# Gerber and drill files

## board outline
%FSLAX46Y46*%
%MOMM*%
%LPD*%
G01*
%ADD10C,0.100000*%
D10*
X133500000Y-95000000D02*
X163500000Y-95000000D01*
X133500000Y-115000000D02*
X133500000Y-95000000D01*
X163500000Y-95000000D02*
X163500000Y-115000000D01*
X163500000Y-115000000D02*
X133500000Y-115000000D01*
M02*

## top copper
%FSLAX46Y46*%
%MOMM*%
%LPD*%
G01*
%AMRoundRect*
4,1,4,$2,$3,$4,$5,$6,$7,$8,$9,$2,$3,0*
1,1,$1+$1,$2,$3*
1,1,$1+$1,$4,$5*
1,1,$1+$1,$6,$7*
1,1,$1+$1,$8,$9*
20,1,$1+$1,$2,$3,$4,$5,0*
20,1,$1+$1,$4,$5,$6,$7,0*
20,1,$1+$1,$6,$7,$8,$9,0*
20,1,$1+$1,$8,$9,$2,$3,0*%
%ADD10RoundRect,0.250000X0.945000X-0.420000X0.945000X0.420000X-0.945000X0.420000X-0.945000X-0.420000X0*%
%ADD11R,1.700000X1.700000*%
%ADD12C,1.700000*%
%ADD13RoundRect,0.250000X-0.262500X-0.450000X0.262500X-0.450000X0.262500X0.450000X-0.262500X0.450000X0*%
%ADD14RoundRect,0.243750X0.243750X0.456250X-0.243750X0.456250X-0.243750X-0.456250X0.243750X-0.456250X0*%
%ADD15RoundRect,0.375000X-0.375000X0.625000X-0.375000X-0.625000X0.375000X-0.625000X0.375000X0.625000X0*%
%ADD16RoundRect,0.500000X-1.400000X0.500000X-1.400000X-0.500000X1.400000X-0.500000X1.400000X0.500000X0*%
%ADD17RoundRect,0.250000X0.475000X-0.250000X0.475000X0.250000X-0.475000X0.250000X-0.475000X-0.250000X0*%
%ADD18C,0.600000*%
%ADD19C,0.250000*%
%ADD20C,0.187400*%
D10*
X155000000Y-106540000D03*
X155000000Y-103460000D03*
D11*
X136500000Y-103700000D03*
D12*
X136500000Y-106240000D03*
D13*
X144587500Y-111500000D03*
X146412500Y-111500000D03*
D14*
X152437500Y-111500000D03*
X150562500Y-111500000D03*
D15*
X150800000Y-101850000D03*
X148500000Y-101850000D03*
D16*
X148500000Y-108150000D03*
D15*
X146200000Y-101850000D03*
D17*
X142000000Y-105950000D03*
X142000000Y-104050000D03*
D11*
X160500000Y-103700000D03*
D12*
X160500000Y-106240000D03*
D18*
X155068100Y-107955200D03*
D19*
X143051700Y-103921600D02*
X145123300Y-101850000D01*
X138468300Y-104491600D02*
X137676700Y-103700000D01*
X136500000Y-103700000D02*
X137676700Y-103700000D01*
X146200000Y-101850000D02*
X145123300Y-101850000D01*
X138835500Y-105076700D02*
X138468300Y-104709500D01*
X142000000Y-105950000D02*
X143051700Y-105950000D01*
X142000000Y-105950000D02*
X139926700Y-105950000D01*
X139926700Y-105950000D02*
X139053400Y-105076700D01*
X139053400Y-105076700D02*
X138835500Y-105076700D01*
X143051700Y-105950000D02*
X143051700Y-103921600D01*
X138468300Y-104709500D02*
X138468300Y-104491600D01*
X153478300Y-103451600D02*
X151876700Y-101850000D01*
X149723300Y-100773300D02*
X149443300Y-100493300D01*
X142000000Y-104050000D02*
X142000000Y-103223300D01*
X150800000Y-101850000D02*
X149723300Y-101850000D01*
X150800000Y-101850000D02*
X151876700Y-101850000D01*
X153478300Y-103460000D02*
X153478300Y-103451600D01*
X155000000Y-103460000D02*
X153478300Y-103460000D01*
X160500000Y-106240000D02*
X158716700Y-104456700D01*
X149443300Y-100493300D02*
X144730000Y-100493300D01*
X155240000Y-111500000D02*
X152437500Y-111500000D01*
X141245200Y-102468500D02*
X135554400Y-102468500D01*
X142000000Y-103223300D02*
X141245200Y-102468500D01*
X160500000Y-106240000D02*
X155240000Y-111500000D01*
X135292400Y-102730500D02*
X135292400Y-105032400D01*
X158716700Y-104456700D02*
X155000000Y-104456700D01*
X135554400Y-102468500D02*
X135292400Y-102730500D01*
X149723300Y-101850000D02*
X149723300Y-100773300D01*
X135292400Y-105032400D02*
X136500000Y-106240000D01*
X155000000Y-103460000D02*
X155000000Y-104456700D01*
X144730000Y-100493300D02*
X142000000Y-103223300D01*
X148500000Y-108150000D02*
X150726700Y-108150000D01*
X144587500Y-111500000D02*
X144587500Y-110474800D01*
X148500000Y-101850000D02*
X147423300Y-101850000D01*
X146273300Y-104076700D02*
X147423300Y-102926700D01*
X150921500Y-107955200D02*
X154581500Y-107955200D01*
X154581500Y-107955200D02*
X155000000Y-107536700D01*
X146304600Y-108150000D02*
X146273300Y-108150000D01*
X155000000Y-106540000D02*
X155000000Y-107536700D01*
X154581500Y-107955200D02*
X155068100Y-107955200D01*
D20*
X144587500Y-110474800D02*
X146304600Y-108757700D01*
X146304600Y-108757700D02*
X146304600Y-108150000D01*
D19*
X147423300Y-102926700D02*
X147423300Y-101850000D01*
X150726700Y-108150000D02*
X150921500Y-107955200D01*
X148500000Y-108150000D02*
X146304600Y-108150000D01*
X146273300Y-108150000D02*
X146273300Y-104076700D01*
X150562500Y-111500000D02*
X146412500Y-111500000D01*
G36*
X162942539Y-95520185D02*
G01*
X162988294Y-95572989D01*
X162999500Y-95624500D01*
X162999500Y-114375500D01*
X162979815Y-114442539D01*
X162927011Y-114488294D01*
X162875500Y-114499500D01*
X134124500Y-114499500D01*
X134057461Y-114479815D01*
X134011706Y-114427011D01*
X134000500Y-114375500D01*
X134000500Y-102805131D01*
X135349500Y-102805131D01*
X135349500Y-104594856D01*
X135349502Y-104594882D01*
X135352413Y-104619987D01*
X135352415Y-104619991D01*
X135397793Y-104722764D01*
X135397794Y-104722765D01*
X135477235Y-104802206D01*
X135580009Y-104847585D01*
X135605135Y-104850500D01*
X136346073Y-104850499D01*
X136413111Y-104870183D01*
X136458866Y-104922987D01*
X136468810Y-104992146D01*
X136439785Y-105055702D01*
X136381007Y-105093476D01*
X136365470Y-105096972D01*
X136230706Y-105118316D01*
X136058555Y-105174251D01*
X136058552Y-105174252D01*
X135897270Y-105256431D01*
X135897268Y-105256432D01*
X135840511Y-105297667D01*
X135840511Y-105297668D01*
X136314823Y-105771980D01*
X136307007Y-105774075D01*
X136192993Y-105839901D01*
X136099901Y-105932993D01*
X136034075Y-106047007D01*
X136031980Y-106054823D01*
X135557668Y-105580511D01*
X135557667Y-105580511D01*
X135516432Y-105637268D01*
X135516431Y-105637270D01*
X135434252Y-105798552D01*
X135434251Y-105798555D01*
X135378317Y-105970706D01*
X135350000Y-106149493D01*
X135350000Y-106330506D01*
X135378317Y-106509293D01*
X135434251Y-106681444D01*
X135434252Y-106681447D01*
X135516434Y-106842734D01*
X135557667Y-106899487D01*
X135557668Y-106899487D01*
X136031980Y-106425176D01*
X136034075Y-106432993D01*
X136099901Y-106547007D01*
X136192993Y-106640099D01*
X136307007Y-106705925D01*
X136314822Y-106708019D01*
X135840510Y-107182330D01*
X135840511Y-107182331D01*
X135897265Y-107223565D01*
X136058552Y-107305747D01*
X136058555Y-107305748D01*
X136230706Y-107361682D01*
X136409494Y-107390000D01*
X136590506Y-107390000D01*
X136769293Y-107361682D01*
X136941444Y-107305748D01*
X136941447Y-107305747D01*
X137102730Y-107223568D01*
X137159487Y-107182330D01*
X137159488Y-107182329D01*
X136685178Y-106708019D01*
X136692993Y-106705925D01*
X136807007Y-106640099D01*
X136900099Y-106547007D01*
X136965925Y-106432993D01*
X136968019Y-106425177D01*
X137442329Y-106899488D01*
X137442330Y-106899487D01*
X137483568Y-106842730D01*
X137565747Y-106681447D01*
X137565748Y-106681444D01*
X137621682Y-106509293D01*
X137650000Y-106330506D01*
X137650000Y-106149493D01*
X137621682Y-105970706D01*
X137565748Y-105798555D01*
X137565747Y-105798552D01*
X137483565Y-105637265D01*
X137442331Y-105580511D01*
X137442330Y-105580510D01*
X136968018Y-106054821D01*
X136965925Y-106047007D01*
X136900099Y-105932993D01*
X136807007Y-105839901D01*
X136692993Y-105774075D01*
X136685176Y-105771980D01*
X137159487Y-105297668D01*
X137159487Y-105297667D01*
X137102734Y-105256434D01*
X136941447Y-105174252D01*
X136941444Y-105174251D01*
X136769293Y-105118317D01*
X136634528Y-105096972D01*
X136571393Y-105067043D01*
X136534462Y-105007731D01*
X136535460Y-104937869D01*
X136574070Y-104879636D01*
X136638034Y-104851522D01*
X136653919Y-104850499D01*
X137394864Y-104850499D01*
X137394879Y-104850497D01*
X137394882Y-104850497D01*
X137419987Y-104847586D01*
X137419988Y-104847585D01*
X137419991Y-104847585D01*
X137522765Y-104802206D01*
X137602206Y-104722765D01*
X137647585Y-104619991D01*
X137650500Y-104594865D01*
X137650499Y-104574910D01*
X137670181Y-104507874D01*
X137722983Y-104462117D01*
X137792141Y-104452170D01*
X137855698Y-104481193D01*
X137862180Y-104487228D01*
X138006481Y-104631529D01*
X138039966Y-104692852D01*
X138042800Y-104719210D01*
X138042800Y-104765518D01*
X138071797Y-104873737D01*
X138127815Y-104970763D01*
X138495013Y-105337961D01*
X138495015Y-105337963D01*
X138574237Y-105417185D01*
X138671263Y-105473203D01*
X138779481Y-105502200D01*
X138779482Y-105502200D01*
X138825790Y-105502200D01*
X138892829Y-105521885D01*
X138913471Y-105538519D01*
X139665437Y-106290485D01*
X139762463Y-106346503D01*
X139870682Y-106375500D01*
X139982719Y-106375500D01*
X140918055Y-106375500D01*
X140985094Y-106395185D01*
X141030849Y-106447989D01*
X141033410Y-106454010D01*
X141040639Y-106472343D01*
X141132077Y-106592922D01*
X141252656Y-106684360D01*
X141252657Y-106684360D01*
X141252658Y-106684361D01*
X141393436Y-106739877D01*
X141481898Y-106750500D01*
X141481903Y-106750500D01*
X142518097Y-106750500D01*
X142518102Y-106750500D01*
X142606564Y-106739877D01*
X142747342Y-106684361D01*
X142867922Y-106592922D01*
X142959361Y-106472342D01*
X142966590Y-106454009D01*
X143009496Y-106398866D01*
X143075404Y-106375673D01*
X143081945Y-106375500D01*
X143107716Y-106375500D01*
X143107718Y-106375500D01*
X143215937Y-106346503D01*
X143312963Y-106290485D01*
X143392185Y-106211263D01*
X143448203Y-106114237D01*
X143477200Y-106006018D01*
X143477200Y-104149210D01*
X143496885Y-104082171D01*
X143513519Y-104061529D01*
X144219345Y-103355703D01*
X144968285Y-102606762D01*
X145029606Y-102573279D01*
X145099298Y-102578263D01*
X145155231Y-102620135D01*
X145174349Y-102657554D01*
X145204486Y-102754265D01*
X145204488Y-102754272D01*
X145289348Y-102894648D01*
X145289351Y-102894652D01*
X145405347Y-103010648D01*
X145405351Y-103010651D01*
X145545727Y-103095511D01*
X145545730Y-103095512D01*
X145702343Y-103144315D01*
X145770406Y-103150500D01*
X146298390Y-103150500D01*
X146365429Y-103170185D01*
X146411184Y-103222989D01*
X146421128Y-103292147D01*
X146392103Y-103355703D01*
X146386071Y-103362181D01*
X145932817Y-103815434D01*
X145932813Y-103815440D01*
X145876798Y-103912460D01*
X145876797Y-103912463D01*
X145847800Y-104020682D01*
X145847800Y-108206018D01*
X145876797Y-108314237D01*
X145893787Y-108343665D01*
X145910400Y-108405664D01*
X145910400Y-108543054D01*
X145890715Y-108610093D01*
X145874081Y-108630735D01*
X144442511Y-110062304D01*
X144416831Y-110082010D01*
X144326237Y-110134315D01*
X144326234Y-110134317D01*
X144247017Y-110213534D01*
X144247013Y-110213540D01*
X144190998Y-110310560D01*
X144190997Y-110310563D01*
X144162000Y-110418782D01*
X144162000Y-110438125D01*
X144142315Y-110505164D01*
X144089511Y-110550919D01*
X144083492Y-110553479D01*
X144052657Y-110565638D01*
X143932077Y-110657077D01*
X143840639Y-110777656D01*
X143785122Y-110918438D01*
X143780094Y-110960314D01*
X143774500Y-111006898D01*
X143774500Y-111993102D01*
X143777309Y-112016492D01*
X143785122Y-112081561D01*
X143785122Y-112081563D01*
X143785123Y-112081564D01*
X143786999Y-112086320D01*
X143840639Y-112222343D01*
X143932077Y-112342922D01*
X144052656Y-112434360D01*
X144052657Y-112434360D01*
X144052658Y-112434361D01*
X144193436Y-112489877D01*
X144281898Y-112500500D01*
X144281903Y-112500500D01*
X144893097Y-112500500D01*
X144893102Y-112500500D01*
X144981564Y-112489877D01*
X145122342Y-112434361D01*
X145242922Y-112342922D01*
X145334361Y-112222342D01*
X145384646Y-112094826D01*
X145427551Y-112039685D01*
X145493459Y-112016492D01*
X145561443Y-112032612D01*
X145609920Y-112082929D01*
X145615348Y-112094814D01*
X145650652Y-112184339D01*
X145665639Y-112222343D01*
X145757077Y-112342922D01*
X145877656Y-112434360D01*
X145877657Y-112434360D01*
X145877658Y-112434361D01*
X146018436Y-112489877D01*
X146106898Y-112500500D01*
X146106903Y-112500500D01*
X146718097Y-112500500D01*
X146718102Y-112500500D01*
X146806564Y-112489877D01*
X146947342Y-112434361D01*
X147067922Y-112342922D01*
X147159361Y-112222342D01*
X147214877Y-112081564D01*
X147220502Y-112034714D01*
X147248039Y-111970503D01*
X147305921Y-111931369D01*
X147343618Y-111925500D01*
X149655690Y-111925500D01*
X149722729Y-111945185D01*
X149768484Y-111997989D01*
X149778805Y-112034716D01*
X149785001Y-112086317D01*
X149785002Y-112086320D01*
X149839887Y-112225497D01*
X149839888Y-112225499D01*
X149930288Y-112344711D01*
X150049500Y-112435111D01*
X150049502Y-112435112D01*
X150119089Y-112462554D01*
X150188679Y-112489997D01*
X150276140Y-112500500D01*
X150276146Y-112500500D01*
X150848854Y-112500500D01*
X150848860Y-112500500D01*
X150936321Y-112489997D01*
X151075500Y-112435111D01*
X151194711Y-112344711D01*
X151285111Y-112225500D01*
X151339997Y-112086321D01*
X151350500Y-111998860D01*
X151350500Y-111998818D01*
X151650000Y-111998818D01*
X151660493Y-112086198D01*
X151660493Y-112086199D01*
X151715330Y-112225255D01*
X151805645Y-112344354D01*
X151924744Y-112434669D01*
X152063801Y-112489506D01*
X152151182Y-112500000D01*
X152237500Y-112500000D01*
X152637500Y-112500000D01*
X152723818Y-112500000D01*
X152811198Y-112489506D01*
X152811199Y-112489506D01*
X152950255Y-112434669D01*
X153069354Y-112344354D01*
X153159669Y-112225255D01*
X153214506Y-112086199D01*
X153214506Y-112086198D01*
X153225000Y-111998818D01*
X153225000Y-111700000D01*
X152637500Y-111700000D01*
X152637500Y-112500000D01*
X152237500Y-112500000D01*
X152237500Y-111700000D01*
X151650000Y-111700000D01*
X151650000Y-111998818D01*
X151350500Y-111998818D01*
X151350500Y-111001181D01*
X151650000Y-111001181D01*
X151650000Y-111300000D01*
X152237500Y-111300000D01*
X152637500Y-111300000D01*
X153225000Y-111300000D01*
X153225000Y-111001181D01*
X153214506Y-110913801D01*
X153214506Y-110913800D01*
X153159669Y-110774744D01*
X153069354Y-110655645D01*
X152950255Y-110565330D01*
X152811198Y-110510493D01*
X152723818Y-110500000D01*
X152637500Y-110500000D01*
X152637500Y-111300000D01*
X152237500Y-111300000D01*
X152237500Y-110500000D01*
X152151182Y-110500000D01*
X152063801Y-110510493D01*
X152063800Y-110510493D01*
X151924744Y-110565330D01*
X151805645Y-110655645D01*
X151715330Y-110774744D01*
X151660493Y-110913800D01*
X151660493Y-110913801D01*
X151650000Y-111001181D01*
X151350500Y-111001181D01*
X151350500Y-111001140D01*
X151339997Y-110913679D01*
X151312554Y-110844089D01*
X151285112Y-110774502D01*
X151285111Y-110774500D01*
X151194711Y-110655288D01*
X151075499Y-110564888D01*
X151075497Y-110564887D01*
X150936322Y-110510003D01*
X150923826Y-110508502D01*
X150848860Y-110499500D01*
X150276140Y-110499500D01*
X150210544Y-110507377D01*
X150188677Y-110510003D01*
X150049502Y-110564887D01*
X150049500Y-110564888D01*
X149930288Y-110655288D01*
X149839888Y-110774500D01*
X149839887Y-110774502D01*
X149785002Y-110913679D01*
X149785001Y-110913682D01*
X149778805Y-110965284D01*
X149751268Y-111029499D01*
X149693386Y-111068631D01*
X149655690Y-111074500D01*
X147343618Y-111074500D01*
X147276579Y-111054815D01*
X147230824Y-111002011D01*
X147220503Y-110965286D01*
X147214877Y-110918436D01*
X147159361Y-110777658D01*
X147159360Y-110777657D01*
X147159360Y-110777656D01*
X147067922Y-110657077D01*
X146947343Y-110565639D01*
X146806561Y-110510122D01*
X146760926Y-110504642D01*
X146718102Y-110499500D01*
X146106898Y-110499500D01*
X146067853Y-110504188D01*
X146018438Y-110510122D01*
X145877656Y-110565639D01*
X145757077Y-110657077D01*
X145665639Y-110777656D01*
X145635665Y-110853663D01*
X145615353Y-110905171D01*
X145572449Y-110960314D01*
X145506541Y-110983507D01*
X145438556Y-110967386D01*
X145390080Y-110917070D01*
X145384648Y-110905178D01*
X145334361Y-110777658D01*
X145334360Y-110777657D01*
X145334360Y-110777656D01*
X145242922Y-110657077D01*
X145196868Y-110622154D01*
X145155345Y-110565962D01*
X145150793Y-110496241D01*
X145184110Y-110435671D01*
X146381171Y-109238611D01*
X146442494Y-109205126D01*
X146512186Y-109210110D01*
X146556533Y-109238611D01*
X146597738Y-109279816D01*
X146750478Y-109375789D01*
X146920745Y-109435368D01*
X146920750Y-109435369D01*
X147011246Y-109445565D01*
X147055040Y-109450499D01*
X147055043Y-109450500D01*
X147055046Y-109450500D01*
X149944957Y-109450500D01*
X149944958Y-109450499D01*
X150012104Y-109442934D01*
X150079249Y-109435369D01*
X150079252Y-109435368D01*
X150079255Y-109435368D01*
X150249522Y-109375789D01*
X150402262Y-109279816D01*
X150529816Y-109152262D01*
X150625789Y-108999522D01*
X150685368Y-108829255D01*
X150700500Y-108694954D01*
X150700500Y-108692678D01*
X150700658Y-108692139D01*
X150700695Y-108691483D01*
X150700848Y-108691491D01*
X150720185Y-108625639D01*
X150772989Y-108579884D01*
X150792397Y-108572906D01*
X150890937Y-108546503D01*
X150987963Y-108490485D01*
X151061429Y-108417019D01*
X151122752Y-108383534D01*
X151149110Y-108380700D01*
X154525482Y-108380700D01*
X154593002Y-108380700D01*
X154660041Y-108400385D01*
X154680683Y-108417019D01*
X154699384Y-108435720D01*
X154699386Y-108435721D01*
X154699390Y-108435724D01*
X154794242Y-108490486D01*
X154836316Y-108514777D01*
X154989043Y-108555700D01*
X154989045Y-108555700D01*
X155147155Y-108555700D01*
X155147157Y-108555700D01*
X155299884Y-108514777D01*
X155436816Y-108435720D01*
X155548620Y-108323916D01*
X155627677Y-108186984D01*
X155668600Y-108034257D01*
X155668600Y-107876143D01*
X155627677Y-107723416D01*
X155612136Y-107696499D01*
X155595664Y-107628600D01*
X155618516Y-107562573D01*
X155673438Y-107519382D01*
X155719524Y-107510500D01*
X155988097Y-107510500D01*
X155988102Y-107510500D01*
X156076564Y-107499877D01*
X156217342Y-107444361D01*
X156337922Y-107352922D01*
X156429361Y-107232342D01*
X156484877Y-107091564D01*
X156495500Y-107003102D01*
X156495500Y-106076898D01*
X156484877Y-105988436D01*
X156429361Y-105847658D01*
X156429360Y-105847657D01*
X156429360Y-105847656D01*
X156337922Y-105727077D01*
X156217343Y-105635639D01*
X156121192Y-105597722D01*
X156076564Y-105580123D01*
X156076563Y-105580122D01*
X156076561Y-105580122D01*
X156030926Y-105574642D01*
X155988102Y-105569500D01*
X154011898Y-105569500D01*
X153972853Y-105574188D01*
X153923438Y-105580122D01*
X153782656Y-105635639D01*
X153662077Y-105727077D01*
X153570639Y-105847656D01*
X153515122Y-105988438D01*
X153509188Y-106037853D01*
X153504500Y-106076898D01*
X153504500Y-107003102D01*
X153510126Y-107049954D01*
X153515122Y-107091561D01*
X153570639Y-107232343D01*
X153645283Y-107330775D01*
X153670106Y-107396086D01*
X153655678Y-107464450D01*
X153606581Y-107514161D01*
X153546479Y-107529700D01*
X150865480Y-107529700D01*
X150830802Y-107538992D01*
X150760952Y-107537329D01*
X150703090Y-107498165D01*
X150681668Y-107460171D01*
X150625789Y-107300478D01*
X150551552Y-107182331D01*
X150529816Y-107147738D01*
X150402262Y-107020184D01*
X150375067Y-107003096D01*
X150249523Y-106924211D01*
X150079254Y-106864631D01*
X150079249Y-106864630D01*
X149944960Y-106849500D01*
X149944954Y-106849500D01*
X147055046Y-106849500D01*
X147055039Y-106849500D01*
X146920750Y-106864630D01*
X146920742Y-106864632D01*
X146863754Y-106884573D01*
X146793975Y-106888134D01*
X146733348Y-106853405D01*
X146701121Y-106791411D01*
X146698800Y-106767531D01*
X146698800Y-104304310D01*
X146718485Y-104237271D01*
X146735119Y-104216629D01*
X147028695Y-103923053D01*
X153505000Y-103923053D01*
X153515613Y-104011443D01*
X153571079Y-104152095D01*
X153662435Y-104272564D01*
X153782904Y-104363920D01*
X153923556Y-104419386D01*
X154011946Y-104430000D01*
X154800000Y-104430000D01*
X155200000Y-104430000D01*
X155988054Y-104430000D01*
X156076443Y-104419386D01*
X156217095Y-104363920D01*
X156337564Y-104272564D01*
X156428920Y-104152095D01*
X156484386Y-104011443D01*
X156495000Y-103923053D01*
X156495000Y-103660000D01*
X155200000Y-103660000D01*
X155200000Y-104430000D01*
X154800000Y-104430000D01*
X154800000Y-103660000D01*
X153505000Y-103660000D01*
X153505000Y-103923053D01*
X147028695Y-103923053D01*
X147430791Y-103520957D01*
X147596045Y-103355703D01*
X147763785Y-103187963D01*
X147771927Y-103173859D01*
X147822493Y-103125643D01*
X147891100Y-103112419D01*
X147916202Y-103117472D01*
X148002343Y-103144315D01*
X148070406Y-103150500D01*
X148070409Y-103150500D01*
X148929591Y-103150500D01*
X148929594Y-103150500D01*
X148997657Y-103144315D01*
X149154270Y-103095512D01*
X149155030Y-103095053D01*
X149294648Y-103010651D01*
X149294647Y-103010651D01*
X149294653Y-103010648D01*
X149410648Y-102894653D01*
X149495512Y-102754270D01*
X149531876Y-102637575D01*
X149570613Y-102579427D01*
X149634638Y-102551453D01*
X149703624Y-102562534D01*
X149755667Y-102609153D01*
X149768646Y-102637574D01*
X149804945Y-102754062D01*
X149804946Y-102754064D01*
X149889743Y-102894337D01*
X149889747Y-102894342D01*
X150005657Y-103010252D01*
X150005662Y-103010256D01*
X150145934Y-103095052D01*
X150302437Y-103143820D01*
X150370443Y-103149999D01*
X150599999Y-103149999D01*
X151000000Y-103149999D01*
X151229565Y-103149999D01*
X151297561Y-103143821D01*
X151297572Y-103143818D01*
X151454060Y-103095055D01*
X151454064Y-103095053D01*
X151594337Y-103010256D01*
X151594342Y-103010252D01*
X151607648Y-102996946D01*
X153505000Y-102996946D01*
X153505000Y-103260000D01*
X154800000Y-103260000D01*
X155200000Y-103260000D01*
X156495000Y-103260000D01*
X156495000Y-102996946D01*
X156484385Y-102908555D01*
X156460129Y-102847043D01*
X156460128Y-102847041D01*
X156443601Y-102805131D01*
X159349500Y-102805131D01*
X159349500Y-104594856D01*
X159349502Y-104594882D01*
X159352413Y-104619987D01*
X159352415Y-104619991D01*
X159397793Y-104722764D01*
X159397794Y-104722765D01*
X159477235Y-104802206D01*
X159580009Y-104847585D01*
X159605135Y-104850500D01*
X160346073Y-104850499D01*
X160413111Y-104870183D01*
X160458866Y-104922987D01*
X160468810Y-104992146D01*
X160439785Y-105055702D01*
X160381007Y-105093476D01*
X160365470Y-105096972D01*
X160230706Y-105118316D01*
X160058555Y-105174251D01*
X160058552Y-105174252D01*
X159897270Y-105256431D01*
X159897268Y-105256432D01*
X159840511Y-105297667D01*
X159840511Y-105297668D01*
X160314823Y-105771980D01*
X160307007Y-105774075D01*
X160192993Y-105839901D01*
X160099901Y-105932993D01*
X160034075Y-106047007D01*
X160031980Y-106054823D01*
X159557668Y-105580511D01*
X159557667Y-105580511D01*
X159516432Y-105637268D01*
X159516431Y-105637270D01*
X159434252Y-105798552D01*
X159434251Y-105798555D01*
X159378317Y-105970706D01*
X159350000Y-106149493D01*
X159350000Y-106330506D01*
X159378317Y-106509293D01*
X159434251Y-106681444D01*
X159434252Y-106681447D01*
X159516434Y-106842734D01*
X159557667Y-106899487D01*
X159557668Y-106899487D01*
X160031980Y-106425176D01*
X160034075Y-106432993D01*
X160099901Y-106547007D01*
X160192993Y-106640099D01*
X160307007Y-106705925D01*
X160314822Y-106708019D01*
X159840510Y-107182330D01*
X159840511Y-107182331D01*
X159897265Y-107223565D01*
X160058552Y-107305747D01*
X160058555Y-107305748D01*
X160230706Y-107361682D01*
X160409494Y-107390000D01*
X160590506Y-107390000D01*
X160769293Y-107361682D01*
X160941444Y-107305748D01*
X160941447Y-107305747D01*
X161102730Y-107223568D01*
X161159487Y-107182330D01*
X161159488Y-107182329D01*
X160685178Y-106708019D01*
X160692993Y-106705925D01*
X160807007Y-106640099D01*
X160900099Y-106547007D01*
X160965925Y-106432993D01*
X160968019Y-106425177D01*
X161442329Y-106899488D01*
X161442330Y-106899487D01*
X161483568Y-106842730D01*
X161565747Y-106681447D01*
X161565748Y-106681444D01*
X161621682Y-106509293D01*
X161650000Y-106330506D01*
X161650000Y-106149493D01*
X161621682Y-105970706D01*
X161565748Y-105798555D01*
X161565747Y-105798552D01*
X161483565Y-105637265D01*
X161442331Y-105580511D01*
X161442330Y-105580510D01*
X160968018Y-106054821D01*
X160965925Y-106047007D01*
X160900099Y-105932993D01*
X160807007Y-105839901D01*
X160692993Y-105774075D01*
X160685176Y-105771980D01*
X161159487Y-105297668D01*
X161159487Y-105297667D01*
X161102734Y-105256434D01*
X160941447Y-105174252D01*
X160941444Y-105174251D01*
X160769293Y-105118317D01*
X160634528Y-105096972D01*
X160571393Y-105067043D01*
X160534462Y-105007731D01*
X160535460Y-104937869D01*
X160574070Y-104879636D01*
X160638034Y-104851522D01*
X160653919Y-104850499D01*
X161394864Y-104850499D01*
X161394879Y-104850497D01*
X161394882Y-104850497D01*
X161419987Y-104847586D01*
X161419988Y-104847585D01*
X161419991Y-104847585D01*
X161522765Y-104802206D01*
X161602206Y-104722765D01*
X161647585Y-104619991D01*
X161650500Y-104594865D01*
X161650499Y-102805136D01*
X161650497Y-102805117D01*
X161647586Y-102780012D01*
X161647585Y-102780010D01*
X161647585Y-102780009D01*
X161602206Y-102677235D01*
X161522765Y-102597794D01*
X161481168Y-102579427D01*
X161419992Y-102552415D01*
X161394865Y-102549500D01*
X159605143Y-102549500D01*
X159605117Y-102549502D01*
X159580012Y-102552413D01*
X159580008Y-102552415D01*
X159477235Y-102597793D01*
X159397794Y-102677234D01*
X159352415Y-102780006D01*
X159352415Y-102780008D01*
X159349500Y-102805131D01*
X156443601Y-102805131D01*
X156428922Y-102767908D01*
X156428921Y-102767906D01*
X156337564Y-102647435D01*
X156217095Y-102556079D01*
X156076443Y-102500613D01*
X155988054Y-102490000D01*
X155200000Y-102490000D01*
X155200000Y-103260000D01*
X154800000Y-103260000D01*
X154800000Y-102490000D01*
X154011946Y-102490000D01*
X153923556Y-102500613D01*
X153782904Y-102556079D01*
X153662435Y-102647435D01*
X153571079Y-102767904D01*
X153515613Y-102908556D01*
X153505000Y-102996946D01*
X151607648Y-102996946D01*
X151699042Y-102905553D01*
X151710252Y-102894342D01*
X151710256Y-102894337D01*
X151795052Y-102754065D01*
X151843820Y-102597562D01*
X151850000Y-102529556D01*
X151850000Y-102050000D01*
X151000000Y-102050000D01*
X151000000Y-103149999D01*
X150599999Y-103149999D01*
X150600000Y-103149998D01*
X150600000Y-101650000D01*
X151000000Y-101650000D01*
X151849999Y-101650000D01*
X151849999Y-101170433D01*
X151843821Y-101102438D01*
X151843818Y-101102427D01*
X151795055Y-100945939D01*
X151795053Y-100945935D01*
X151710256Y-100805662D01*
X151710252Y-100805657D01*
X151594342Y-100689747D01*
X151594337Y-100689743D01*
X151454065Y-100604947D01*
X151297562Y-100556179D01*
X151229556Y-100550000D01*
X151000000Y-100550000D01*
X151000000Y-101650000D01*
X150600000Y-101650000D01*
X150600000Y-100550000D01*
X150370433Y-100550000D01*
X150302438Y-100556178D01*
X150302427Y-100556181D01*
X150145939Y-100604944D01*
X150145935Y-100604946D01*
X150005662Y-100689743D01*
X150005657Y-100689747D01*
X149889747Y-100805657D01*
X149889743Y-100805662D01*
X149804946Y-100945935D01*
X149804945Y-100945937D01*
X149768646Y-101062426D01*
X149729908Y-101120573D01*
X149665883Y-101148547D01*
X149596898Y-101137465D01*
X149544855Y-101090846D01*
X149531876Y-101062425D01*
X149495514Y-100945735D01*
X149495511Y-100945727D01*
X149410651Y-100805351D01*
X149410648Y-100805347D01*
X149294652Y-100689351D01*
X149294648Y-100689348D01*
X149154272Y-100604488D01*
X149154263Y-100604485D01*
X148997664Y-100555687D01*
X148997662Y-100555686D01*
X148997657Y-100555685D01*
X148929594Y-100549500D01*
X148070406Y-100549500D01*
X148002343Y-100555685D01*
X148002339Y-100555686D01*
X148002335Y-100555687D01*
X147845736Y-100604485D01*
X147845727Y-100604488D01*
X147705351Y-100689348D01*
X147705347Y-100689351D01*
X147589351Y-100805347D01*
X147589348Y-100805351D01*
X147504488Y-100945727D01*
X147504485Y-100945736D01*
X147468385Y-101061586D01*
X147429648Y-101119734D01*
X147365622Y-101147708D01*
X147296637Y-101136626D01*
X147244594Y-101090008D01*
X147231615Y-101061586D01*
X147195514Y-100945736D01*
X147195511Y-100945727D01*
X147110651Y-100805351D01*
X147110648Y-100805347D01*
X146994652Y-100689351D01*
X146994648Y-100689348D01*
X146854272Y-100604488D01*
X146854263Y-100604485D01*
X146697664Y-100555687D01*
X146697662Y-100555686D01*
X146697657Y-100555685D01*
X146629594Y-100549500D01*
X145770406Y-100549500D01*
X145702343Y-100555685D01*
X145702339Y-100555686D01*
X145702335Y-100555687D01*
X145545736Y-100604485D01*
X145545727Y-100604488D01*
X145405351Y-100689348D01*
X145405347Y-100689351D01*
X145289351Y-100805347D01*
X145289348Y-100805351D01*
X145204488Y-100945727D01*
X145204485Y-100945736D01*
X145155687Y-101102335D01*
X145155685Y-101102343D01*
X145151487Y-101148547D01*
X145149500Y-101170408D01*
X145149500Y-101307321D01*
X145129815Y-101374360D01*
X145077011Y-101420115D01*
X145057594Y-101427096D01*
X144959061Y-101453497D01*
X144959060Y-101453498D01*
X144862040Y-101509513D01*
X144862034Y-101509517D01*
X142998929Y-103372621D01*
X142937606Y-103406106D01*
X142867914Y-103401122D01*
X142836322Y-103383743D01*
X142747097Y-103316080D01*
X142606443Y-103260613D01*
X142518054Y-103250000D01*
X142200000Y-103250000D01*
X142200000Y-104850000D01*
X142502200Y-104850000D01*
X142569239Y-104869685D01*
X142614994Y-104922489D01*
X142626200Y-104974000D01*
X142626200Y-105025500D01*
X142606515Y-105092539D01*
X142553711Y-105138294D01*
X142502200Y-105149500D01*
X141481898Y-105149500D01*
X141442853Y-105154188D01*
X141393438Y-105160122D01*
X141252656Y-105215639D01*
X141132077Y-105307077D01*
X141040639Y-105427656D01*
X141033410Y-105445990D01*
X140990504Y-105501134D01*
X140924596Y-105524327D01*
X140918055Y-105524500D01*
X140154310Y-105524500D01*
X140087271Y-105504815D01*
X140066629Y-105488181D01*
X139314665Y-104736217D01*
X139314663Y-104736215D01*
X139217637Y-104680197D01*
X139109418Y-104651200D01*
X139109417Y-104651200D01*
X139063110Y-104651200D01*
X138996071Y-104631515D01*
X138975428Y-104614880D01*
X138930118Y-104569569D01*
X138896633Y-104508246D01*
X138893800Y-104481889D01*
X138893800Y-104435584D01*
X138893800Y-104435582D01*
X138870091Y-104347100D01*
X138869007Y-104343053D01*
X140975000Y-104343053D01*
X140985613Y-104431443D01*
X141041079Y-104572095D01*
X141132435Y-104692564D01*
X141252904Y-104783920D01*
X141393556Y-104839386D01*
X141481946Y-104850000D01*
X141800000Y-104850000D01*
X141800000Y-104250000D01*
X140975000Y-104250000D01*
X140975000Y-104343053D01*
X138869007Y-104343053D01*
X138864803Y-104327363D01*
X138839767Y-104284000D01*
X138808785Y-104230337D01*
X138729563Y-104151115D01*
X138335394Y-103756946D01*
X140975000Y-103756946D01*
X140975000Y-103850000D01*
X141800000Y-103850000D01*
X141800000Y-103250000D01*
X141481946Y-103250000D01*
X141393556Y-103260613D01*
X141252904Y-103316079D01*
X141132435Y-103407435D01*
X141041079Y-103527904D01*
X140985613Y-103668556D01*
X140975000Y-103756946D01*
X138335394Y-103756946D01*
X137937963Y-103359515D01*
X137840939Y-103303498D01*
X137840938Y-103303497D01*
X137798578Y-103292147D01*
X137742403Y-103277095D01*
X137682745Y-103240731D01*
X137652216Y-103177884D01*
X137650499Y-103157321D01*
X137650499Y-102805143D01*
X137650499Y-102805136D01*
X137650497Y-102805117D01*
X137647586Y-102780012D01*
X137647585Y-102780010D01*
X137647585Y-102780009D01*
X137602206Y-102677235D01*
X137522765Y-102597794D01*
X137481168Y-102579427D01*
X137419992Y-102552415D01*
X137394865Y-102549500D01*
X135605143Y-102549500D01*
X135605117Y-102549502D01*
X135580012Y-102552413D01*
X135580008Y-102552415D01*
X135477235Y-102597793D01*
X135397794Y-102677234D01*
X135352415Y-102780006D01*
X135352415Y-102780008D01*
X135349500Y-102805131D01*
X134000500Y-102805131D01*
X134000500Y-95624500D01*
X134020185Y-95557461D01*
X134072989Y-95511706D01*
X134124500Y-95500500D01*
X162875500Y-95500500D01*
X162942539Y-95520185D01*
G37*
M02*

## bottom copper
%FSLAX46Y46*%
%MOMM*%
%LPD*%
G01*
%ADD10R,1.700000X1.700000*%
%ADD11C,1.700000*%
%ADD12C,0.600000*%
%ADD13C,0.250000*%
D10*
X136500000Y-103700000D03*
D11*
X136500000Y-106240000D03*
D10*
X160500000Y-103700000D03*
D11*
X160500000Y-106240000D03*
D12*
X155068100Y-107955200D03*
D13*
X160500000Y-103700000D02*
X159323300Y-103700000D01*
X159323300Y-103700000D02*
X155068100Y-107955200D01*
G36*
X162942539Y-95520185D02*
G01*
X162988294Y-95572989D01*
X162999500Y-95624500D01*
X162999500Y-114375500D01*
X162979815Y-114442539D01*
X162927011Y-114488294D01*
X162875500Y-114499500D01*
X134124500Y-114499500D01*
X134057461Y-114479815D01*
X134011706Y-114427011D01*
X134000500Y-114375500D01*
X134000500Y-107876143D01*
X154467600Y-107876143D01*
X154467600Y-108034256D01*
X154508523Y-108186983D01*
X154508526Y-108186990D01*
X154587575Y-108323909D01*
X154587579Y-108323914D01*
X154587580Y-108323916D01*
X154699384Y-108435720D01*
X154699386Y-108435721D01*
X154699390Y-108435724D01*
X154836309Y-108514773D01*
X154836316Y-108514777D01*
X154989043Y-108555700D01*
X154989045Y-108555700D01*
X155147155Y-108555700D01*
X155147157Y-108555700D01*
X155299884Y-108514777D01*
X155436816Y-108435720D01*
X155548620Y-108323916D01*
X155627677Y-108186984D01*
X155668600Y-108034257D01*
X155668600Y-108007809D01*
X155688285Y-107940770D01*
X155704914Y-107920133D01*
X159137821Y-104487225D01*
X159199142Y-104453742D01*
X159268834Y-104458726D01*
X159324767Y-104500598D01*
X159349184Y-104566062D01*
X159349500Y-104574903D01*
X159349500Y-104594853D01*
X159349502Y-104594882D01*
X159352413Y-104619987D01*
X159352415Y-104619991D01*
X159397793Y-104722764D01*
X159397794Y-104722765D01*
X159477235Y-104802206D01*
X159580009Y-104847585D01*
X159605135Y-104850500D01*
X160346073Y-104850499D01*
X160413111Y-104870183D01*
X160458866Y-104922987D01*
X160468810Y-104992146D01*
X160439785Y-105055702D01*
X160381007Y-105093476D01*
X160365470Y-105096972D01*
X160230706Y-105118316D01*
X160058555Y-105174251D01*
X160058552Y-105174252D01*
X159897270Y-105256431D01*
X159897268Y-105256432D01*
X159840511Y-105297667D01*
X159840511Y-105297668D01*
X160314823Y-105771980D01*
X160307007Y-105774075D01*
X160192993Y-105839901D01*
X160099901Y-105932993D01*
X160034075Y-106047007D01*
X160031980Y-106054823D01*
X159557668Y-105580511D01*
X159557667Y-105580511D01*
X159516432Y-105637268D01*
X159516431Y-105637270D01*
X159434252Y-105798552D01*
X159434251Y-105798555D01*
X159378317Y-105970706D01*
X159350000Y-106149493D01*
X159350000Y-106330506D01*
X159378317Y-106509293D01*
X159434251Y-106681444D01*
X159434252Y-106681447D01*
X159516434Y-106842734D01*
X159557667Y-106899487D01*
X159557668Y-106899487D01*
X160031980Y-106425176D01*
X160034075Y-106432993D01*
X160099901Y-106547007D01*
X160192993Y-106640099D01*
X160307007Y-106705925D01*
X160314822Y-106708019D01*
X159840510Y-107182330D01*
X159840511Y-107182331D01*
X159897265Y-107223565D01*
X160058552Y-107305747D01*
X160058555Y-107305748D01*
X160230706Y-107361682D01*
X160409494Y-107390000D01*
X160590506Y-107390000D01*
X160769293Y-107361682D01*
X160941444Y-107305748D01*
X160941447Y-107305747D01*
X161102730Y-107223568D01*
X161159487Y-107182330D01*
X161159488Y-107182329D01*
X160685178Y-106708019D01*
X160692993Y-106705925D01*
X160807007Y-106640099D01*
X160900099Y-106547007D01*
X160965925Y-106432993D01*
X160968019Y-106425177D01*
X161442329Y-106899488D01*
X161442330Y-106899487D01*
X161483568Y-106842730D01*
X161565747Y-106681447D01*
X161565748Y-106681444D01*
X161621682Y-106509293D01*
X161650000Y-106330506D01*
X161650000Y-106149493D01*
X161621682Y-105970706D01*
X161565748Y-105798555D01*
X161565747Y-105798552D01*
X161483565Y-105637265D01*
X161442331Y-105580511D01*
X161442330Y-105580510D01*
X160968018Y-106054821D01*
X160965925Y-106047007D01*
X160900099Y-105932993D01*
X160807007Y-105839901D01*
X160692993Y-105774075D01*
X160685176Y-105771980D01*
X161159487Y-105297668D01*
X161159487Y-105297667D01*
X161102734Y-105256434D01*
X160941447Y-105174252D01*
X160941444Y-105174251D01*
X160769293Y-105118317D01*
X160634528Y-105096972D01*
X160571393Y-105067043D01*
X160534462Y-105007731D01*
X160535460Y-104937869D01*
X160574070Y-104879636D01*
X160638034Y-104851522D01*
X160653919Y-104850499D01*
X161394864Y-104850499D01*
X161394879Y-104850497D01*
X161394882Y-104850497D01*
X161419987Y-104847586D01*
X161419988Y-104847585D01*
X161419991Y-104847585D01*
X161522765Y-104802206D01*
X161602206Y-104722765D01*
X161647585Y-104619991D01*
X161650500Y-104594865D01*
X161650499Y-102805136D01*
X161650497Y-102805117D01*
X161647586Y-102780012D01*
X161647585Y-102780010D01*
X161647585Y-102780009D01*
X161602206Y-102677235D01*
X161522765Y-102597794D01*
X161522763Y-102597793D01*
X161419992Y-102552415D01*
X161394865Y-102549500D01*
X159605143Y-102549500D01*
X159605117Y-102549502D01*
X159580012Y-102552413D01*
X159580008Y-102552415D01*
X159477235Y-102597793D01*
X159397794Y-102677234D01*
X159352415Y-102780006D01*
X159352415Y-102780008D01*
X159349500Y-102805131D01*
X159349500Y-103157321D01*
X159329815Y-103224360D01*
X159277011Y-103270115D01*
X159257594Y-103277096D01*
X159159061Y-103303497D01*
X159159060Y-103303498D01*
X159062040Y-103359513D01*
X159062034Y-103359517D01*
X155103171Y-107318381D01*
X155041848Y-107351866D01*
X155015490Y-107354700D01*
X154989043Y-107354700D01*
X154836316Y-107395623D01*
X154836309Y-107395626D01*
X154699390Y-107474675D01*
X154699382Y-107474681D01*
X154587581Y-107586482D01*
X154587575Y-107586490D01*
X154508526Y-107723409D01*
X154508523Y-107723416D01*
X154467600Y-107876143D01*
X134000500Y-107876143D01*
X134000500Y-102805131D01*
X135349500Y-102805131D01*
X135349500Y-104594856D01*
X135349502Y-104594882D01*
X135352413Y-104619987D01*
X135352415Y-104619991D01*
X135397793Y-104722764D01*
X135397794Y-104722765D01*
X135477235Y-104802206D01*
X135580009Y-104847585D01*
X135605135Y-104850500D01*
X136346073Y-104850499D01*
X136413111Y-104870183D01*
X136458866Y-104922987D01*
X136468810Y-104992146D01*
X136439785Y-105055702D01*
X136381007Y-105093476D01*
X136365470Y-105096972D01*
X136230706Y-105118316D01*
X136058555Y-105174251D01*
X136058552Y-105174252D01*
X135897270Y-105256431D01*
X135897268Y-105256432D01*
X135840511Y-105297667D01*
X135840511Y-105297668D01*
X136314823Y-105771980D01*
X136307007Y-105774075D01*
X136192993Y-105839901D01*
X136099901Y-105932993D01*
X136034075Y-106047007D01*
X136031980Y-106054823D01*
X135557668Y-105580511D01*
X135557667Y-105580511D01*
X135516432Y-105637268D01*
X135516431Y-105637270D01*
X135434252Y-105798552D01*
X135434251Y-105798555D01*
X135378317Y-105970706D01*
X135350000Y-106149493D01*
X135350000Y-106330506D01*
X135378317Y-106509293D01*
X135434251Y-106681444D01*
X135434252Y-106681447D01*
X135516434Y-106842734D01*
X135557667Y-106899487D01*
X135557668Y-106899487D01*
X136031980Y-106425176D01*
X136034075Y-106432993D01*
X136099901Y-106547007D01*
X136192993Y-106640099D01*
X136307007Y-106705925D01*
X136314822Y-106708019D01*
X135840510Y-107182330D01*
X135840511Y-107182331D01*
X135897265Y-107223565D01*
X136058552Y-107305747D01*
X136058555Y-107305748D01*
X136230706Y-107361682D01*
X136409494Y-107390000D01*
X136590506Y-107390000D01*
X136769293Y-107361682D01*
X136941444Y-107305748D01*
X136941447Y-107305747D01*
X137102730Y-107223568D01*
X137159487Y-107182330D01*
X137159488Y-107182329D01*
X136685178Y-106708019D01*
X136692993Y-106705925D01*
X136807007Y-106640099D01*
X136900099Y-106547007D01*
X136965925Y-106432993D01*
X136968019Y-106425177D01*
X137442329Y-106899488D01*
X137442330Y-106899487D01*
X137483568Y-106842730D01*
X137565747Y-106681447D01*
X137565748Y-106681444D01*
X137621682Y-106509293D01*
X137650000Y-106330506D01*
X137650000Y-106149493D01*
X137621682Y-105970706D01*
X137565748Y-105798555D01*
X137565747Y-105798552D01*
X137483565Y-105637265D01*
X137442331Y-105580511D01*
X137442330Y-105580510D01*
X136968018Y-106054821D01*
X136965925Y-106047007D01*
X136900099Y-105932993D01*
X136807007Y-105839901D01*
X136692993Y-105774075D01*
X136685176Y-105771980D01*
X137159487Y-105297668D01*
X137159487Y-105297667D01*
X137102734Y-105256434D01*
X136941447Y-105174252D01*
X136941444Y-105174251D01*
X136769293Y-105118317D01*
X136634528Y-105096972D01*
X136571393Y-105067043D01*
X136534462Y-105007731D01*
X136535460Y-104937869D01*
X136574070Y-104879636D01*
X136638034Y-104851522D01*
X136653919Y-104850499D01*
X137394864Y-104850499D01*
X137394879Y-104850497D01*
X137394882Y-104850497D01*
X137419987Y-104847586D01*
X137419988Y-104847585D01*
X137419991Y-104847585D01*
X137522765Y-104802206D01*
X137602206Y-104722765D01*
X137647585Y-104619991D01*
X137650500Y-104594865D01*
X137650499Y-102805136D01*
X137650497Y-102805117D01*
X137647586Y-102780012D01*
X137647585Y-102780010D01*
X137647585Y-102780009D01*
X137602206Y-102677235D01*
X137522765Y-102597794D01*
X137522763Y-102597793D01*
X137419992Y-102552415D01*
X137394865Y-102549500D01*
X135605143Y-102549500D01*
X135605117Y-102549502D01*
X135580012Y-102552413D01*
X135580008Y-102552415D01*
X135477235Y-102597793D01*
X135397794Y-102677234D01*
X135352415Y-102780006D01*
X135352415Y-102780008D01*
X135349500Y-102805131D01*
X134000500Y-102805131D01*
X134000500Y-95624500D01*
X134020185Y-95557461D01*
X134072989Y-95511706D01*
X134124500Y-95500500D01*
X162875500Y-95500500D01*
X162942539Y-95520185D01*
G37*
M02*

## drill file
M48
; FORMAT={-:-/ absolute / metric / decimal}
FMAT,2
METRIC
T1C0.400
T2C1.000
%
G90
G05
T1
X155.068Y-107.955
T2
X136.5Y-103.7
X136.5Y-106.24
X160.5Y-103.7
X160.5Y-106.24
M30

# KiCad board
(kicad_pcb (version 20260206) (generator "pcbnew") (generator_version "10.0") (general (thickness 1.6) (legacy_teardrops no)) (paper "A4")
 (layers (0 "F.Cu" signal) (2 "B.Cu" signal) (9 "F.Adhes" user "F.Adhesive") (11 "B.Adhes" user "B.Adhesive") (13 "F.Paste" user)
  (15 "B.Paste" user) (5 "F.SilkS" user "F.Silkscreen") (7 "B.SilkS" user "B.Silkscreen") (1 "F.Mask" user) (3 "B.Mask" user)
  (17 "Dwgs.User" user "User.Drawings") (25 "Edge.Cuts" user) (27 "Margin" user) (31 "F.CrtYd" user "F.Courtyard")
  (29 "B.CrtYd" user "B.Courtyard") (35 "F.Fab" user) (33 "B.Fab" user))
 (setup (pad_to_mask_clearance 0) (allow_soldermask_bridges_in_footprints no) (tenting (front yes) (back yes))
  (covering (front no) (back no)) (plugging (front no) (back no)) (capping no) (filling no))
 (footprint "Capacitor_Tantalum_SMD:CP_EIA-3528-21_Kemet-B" (layer "F.Cu") (at 155 105 90)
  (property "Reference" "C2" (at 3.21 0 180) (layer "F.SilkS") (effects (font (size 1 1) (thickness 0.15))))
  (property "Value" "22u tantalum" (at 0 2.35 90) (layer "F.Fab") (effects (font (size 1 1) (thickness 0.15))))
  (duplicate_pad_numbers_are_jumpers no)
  (pad "1" smd roundrect (at -1.54 0 90) (size 1.34 2.39) (layers "F.Cu" "F.Mask" "F.Paste") (roundrect_rratio 0.186567) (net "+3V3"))
  (pad "2" smd roundrect (at 1.54 0 90) (size 1.34 2.39) (layers "F.Cu" "F.Mask" "F.Paste") (roundrect_rratio 0.186567) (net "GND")))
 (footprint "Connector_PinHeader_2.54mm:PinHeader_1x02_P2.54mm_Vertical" (layer "F.Cu") (at 136.5 103.7)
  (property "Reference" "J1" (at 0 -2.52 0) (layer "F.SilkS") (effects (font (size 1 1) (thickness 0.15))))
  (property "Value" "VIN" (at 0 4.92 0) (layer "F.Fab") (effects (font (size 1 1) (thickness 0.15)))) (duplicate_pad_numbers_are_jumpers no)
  (pad "1" thru_hole rect (at 0 0) (size 1.7 1.7) (drill 1) (layers "*.Cu" "*.Mask") (remove_unused_layers no) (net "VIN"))
  (pad "2" thru_hole circle (at 0 2.54) (size 1.7 1.7) (drill 1) (layers "*.Cu" "*.Mask") (remove_unused_layers no) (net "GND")))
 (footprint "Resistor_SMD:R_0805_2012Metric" (layer "F.Cu") (at 145.5 111.5)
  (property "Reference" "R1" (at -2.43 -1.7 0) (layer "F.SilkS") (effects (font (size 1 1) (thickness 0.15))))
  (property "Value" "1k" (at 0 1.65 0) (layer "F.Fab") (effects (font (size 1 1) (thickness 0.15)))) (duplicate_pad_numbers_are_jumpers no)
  (pad "1" smd roundrect (at -0.9125 0) (size 1.025 1.4) (layers "F.Cu" "F.Mask" "F.Paste") (roundrect_rratio 0.243902) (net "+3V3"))
  (pad "2" smd roundrect (at 0.9125 0) (size 1.025 1.4) (layers "F.Cu" "F.Mask" "F.Paste") (roundrect_rratio 0.243902) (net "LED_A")))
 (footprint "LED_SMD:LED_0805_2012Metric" (layer "F.Cu") (at 151.5 111.5 180)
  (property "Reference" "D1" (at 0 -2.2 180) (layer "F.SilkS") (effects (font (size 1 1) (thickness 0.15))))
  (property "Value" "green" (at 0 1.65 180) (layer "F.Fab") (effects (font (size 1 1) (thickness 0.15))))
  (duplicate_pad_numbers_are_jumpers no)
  (pad "1" smd roundrect (at -0.9375 0 180) (size 0.975 1.4) (layers "F.Cu" "F.Mask" "F.Paste") (roundrect_rratio 0.25) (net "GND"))
  (pad "2" smd roundrect (at 0.9375 0 180) (size 0.975 1.4) (layers "F.Cu" "F.Mask" "F.Paste") (roundrect_rratio 0.25) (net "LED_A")))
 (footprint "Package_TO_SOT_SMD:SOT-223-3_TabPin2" (layer "F.Cu") (at 148.5 105 -90)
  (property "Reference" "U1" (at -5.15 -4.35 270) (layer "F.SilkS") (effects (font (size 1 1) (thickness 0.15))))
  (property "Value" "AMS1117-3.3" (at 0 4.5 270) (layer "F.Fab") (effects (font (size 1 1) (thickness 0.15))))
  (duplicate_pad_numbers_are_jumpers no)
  (pad "1" smd roundrect (at -3.15 -2.3 270) (size 2 1.5) (layers "F.Cu" "F.Mask" "F.Paste") (roundrect_rratio 0.25) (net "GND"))
  (pad "2" smd roundrect (at -3.15 0 270) (size 2 1.5) (layers "F.Cu" "F.Mask" "F.Paste") (roundrect_rratio 0.25) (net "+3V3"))
  (pad "2" smd roundrect (at 3.15 0 270) (size 2 3.8) (layers "F.Cu" "F.Mask" "F.Paste") (roundrect_rratio 0.25) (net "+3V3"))
  (pad "3" smd roundrect (at -3.15 2.3 270) (size 2 1.5) (layers "F.Cu" "F.Mask" "F.Paste") (roundrect_rratio 0.25) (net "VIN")))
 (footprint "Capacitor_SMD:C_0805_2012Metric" (layer "F.Cu") (at 142 105 90)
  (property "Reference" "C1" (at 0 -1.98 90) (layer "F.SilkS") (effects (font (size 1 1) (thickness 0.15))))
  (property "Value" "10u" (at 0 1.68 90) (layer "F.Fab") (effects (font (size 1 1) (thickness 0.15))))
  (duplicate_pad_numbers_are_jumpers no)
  (pad "1" smd roundrect (at -0.95 0 90) (size 1 1.45) (layers "F.Cu" "F.Mask" "F.Paste") (roundrect_rratio 0.25) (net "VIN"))
  (pad "2" smd roundrect (at 0.95 0 90) (size 1 1.45) (layers "F.Cu" "F.Mask" "F.Paste") (roundrect_rratio 0.25) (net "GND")))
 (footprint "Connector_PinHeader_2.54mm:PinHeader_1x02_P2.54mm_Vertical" (layer "F.Cu") (at 160.5 103.7)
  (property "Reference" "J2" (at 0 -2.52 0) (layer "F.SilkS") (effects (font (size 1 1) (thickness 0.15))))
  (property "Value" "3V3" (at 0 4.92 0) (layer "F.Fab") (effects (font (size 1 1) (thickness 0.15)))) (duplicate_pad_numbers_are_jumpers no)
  (pad "1" thru_hole rect (at 0 0) (size 1.7 1.7) (drill 1) (layers "*.Cu" "*.Mask") (remove_unused_layers no) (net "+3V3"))
  (pad "2" thru_hole circle (at 0 2.54) (size 1.7 1.7) (drill 1) (layers "*.Cu" "*.Mask") (remove_unused_layers no) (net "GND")))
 (gr_line (start 133.5 95) (end 163.5 95) (stroke (width 0.1) (type default)) (layer "Edge.Cuts"))
 (gr_line (start 133.5 115) (end 133.5 95) (stroke (width 0.1) (type default)) (layer "Edge.Cuts"))
 (gr_line (start 163.5 95) (end 163.5 115) (stroke (width 0.1) (type default)) (layer "Edge.Cuts"))
 (gr_line (start 163.5 115) (end 133.5 115) (stroke (width 0.1) (type default)) (layer "Edge.Cuts"))
 (segment (start 143.0517 103.9216) (end 145.1233 101.85) (width 0.25) (layer "F.Cu") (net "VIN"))
 (segment (start 138.4683 104.4916) (end 137.6767 103.7) (width 0.25) (layer "F.Cu") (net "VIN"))
 (segment (start 136.5 103.7) (end 137.6767 103.7) (width 0.25) (layer "F.Cu") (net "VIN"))
 (segment (start 146.2 101.85) (end 145.1233 101.85) (width 0.25) (layer "F.Cu") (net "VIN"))
 (segment (start 138.8355 105.0767) (end 138.4683 104.7095) (width 0.25) (layer "F.Cu") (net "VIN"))
 (segment (start 142 105.95) (end 143.0517 105.95) (width 0.25) (layer "F.Cu") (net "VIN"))
 (segment (start 142 105.95) (end 139.9267 105.95) (width 0.25) (layer "F.Cu") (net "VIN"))
 (segment (start 139.9267 105.95) (end 139.0534 105.0767) (width 0.25) (layer "F.Cu") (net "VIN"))
 (segment (start 139.0534 105.0767) (end 138.8355 105.0767) (width 0.25) (layer "F.Cu") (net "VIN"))
 (segment (start 143.0517 105.95) (end 143.0517 103.9216) (width 0.25) (layer "F.Cu") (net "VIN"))
 (segment (start 138.4683 104.7095) (end 138.4683 104.4916) (width 0.25) (layer "F.Cu") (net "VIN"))
 (segment (start 153.4783 103.4516) (end 151.8767 101.85) (width 0.25) (layer "F.Cu") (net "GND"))
 (segment (start 149.7233 100.7733) (end 149.4433 100.4933) (width 0.25) (layer "F.Cu") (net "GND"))
 (segment (start 142 104.05) (end 142 103.2233) (width 0.25) (layer "F.Cu") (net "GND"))
 (segment (start 150.8 101.85) (end 149.7233 101.85) (width 0.25) (layer "F.Cu") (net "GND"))
 (segment (start 150.8 101.85) (end 151.8767 101.85) (width 0.25) (layer "F.Cu") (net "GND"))
 (segment (start 153.4783 103.46) (end 153.4783 103.4516) (width 0.25) (layer "F.Cu") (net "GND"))
 (segment (start 155 103.46) (end 153.4783 103.46) (width 0.25) (layer "F.Cu") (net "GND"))
 (segment (start 160.5 106.24) (end 158.7167 104.4567) (width 0.25) (layer "F.Cu") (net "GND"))
 (segment (start 149.4433 100.4933) (end 144.73 100.4933) (width 0.25) (layer "F.Cu") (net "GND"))
 (segment (start 155.24 111.5) (end 152.4375 111.5) (width 0.25) (layer "F.Cu") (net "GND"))
 (segment (start 141.2452 102.4685) (end 135.5544 102.4685) (width 0.25) (layer "F.Cu") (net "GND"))
 (segment (start 142 103.2233) (end 141.2452 102.4685) (width 0.25) (layer "F.Cu") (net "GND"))
 (segment (start 160.5 106.24) (end 155.24 111.5) (width 0.25) (layer "F.Cu") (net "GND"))
 (segment (start 135.2924 102.7305) (end 135.2924 105.0324) (width 0.25) (layer "F.Cu") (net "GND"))
 (segment (start 158.7167 104.4567) (end 155 104.4567) (width 0.25) (layer "F.Cu") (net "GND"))
 (segment (start 135.5544 102.4685) (end 135.2924 102.7305) (width 0.25) (layer "F.Cu") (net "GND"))
 (segment (start 149.7233 101.85) (end 149.7233 100.7733) (width 0.25) (layer "F.Cu") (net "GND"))
 (segment (start 135.2924 105.0324) (end 136.5 106.24) (width 0.25) (layer "F.Cu") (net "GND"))
 (segment (start 155 103.46) (end 155 104.4567) (width 0.25) (layer "F.Cu") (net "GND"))
 (segment (start 144.73 100.4933) (end 142 103.2233) (width 0.25) (layer "F.Cu") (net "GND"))
 (segment (start 148.5 108.15) (end 150.7267 108.15) (width 0.25) (layer "F.Cu") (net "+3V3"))
 (segment (start 144.5875 111.5) (end 144.5875 110.4748) (width 0.25) (layer "F.Cu") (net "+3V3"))
 (segment (start 148.5 101.85) (end 147.4233 101.85) (width 0.25) (layer "F.Cu") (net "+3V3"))
 (segment (start 146.2733 104.0767) (end 147.4233 102.9267) (width 0.25) (layer "F.Cu") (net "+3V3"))
 (segment (start 150.9215 107.9552) (end 154.5815 107.9552) (width 0.25) (layer "F.Cu") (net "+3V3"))
 (segment (start 154.5815 107.9552) (end 155 107.5367) (width 0.25) (layer "F.Cu") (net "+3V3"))
 (segment (start 146.3046 108.15) (end 146.2733 108.15) (width 0.25) (layer "F.Cu") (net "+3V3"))
 (segment (start 155 106.54) (end 155 107.5367) (width 0.25) (layer "F.Cu") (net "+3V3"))
 (segment (start 154.5815 107.9552) (end 155.0681 107.9552) (width 0.25) (layer "F.Cu") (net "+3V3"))
 (segment (start 144.5875 110.4748) (end 146.3046 108.7577) (width 0.1874) (layer "F.Cu") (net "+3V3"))
 (segment (start 146.3046 108.7577) (end 146.3046 108.15) (width 0.1874) (layer "F.Cu") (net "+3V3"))
 (segment (start 147.4233 102.9267) (end 147.4233 101.85) (width 0.25) (layer "F.Cu") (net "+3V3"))
 (segment (start 150.7267 108.15) (end 150.9215 107.9552) (width 0.25) (layer "F.Cu") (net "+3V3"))
 (segment (start 148.5 108.15) (end 146.3046 108.15) (width 0.25) (layer "F.Cu") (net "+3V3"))
 (segment (start 146.2733 108.15) (end 146.2733 104.0767) (width 0.25) (layer "F.Cu") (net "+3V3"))
 (via (at 155.0681 107.9552) (size 0.6) (drill 0.4) (layers "F.Cu" "B.Cu") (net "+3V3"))
 (segment (start 160.5 103.7) (end 159.3233 103.7) (width 0.25) (layer "B.Cu") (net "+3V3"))
 (segment (start 159.3233 103.7) (end 155.0681 107.9552) (width 0.25) (layer "B.Cu") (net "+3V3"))
 (segment (start 150.5625 111.5) (end 146.4125 111.5) (width 0.25) (layer "F.Cu") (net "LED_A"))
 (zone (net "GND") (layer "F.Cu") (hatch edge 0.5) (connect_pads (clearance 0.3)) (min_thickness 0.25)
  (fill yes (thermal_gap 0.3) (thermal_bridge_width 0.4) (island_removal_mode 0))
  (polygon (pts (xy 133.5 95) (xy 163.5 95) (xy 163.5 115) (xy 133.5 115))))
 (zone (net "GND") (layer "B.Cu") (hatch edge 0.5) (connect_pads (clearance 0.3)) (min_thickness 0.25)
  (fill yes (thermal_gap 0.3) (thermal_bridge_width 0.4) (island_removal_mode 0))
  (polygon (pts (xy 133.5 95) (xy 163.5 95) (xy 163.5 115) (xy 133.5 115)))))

